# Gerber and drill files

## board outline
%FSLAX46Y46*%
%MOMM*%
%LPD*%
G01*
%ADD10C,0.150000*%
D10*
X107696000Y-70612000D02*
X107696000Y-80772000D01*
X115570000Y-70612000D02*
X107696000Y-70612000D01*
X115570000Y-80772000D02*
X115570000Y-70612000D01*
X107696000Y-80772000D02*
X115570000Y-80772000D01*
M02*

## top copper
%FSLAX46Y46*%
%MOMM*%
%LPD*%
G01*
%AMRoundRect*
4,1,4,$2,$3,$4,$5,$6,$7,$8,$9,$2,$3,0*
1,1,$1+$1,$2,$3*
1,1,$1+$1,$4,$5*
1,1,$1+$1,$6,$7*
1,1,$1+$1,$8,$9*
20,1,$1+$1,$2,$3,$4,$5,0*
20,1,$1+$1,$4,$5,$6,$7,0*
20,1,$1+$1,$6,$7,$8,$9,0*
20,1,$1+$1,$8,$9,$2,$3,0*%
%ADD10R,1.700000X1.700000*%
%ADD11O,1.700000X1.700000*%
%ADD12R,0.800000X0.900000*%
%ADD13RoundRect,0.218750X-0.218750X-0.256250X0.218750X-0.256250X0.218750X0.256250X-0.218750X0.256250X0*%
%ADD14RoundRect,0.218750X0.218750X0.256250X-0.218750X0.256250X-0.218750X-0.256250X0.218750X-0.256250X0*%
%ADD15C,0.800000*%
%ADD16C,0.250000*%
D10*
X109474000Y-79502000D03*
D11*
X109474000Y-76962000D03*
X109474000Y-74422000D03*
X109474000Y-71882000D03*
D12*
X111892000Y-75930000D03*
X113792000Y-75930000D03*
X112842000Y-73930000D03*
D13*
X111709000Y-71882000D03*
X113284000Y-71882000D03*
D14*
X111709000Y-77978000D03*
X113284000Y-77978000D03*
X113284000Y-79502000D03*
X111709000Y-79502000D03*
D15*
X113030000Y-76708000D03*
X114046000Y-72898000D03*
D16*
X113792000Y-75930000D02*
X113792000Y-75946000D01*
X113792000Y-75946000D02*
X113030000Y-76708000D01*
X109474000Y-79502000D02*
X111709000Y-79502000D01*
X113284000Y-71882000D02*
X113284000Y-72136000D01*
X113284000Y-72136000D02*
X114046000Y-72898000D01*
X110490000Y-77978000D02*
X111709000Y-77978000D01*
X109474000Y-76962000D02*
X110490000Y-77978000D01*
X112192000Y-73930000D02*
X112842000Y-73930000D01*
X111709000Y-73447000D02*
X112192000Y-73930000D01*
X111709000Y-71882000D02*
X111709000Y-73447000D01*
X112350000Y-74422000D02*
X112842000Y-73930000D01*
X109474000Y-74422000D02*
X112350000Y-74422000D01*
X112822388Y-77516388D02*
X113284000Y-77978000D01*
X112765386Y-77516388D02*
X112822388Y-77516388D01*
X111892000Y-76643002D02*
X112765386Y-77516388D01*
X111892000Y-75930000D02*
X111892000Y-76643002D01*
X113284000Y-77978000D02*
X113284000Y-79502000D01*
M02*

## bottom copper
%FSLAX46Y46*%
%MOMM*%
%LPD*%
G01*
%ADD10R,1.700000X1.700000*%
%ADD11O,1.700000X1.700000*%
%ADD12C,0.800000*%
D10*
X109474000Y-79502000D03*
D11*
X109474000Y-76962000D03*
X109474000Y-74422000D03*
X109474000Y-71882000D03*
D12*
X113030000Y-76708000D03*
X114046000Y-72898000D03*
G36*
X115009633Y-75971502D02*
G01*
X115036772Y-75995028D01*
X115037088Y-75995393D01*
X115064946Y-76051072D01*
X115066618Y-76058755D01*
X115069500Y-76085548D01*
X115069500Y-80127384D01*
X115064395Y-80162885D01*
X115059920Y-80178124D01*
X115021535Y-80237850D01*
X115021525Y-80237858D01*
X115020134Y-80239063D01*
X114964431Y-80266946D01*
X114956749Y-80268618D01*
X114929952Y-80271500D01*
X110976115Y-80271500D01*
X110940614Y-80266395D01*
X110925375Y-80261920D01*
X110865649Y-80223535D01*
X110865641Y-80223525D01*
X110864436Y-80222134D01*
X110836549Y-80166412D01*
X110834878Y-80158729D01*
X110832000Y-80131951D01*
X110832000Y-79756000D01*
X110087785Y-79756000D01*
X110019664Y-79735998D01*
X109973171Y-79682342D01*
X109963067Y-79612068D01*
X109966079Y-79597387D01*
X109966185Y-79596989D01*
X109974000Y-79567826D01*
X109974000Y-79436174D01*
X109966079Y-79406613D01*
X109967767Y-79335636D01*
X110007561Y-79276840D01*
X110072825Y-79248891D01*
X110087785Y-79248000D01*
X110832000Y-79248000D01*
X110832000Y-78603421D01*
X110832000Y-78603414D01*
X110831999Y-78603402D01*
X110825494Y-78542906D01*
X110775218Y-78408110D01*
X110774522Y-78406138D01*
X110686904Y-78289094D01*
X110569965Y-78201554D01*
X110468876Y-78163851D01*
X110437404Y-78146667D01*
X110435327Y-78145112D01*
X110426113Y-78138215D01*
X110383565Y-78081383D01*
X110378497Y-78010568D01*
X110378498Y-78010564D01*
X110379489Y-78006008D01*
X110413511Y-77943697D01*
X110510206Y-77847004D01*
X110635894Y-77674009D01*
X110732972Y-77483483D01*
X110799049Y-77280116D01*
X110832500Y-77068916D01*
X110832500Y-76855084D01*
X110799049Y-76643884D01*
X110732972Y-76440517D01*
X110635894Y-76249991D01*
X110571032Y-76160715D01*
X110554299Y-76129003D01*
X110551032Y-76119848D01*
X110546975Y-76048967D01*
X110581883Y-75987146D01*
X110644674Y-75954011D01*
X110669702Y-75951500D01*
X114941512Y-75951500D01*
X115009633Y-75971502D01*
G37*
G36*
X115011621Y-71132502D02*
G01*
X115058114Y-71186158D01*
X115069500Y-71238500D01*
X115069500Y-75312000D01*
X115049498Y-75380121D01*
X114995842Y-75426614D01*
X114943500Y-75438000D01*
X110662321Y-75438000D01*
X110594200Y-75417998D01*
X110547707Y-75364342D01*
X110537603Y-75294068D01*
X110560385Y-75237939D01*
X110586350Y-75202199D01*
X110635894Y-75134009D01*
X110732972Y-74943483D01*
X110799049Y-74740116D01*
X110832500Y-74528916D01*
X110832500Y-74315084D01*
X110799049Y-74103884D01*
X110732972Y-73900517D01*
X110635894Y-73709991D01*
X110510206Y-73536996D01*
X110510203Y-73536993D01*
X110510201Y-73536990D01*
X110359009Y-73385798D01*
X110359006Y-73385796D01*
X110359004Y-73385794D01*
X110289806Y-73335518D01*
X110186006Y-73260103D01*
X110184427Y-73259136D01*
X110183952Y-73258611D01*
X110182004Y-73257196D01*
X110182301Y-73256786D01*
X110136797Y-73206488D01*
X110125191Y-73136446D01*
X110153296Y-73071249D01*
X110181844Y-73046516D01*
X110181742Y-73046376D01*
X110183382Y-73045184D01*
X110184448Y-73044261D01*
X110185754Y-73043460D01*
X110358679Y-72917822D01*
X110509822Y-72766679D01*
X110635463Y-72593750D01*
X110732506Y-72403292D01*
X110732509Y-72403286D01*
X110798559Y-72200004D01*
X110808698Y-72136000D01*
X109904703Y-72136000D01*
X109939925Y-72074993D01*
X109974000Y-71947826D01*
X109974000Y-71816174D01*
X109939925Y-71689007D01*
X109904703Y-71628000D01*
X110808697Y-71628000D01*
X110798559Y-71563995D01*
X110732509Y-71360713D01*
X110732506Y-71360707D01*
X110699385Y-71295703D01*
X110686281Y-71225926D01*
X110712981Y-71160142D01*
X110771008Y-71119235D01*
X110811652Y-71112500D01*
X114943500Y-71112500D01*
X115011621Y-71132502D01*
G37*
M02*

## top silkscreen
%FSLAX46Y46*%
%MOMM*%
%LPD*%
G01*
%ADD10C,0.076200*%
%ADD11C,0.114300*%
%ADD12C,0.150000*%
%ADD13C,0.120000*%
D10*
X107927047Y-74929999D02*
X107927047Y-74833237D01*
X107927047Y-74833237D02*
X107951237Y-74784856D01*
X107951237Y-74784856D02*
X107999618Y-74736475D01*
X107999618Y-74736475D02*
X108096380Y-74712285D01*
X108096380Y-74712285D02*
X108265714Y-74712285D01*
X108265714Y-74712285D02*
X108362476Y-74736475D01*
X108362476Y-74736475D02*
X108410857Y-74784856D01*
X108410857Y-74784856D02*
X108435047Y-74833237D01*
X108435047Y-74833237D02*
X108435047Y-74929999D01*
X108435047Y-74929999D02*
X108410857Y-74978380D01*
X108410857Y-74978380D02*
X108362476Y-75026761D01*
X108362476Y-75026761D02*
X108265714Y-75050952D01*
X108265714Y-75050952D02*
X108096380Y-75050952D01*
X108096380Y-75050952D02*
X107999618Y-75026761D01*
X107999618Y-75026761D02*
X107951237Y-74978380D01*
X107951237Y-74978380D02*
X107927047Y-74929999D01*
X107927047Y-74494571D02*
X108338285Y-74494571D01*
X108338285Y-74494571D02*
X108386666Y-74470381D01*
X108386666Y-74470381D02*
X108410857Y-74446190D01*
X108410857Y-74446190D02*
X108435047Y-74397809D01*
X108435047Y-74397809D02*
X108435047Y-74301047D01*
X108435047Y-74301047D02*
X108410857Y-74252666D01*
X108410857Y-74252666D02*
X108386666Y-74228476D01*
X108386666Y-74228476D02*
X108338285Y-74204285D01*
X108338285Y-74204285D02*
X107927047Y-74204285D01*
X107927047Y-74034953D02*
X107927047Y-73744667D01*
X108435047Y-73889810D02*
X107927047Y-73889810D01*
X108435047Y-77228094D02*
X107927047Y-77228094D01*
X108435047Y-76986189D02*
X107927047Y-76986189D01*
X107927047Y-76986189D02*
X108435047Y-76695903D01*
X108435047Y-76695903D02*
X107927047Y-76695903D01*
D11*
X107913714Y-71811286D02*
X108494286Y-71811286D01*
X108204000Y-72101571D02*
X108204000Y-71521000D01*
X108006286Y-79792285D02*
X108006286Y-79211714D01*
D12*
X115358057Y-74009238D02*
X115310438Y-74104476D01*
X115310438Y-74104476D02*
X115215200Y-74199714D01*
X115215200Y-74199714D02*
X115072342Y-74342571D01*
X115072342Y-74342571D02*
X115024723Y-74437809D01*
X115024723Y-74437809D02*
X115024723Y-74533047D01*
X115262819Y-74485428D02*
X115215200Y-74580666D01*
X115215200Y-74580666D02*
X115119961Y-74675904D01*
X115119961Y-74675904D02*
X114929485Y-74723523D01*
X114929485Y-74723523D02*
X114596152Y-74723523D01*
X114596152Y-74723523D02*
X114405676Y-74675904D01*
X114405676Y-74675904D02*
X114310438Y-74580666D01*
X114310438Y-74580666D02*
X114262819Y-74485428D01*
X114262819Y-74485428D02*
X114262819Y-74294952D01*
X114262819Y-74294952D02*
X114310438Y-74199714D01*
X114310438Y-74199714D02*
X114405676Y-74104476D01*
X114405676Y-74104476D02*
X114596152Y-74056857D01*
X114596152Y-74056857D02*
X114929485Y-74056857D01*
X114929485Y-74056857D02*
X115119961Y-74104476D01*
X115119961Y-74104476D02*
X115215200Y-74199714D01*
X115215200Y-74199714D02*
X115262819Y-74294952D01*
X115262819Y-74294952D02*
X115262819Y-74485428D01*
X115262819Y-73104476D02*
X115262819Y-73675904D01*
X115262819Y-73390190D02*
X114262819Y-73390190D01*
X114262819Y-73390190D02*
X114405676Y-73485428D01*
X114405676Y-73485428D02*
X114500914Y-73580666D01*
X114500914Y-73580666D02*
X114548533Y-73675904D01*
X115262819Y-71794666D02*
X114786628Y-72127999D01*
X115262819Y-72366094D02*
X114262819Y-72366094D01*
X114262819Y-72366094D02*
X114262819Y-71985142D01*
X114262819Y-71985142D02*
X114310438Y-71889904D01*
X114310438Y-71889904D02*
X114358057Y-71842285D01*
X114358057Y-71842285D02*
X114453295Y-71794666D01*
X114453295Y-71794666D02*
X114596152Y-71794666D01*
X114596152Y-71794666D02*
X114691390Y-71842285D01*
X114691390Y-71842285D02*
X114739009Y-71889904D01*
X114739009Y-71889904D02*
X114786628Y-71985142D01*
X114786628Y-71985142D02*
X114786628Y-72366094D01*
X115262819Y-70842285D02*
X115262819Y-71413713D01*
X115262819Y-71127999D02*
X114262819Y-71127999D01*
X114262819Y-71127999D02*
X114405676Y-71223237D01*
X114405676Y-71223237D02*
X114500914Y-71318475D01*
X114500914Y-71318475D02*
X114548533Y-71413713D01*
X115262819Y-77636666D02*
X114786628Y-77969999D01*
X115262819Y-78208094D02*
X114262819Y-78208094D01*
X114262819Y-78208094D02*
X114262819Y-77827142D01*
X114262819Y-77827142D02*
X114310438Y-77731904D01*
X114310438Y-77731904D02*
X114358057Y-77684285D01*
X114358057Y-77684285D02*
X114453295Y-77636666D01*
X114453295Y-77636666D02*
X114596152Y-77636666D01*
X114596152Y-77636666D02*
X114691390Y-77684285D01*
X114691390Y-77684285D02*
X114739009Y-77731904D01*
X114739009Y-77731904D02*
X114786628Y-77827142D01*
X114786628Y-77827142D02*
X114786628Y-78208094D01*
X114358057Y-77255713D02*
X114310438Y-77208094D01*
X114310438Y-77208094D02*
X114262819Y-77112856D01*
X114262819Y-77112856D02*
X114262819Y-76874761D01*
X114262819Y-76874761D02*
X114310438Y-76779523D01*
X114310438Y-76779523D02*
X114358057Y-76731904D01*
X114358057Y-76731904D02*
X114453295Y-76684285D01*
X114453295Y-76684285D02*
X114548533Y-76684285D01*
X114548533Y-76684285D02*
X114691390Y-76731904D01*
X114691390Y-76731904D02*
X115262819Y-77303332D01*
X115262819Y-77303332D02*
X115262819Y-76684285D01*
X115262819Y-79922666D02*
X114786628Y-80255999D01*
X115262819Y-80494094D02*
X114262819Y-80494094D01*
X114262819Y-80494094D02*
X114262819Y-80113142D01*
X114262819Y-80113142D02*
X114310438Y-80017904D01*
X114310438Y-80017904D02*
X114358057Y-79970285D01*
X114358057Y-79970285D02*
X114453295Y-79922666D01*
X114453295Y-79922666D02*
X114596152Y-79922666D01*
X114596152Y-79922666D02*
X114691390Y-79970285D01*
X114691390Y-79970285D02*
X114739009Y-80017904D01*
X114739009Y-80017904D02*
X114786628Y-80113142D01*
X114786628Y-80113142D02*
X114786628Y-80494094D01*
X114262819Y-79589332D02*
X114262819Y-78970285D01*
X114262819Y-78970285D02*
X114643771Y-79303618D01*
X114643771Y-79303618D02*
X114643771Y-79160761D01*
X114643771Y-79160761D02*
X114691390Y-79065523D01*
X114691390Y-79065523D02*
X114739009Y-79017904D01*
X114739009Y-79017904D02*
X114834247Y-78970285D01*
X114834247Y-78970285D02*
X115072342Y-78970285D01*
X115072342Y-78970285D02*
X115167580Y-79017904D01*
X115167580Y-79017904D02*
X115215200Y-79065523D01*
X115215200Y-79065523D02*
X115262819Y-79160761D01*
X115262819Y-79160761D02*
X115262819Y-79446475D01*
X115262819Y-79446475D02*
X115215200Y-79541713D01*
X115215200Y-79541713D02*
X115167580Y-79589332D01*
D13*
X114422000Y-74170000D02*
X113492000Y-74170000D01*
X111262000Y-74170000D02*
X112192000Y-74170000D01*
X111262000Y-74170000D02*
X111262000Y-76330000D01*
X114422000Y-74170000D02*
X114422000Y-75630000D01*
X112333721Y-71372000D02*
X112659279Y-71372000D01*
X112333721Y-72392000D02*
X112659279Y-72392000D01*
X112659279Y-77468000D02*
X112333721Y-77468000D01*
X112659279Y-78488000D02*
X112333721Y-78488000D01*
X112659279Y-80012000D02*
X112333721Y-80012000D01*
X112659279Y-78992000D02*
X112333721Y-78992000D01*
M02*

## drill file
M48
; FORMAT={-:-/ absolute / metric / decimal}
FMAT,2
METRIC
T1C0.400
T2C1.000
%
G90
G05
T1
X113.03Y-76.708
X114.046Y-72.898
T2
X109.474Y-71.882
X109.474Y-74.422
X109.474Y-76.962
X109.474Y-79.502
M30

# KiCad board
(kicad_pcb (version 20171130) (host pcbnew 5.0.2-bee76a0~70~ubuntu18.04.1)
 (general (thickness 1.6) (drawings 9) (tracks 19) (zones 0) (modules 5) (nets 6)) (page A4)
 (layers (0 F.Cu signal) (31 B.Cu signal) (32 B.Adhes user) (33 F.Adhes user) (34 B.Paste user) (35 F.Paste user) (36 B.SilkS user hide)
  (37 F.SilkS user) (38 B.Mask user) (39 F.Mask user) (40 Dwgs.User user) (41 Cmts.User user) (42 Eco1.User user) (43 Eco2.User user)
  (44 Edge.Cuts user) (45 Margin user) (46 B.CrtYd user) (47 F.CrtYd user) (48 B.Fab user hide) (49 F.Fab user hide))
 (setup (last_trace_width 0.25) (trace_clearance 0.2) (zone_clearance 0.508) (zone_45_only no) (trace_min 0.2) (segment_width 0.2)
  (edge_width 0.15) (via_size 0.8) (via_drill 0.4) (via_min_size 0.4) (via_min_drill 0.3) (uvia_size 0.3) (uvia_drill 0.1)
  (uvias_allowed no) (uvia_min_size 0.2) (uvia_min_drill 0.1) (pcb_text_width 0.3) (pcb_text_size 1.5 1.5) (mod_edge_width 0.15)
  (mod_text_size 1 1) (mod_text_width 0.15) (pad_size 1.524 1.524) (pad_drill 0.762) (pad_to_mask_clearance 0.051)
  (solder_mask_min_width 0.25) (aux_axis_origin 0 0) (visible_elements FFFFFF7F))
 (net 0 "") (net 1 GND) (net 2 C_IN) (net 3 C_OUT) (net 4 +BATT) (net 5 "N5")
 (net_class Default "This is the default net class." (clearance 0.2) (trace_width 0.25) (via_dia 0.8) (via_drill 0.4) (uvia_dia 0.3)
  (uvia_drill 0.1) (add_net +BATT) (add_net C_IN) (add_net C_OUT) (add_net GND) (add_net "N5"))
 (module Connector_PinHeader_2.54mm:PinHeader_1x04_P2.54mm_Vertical (layer B.Cu) (at 109.474 79.502)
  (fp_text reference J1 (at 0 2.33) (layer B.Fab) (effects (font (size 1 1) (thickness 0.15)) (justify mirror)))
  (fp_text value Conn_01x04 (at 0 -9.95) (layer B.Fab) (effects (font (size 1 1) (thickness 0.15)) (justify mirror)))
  (pad 1 thru_hole rect (at 0 0) (size 1.7 1.7) (drill 1) (layers *.Cu *.Mask) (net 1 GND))
  (pad 2 thru_hole oval (at 0 -2.54) (size 1.7 1.7) (drill 1) (layers *.Cu *.Mask) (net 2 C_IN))
  (pad 3 thru_hole oval (at 0 -5.08) (size 1.7 1.7) (drill 1) (layers *.Cu *.Mask) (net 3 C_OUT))
  (pad 4 thru_hole oval (at 0 -7.62) (size 1.7 1.7) (drill 1) (layers *.Cu *.Mask) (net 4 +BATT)))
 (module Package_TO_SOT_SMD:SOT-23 (layer F.Cu) (at 112.842 74.93 90)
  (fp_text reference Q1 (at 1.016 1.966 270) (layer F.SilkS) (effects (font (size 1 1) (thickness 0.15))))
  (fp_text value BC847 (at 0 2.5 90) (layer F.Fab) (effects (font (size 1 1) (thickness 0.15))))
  (fp_line (start 0.76 1.58) (end 0.76 0.65) (layer F.SilkS) (width 0.12))
  (fp_line (start 0.76 -1.58) (end 0.76 -0.65) (layer F.SilkS) (width 0.12))
  (fp_line (start 0.76 -1.58) (end -1.4 -1.58) (layer F.SilkS) (width 0.12))
  (fp_line (start 0.76 1.58) (end -0.7 1.58) (layer F.SilkS) (width 0.12))
  (pad 1 smd rect (at -1 -0.95 90) (size 0.9 0.8) (layers F.Cu F.Paste F.Mask) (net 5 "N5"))
  (pad 2 smd rect (at -1 0.95 90) (size 0.9 0.8) (layers F.Cu F.Paste F.Mask) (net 1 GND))
  (pad 3 smd rect (at 1 0 90) (size 0.9 0.8) (layers F.Cu F.Paste F.Mask) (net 3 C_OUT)))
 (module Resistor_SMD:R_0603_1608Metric (layer F.Cu) (at 112.4965 71.882)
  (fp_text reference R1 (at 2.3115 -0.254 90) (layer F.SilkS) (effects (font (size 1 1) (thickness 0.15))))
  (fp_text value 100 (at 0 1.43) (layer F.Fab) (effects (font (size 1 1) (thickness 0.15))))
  (fp_line (start -0.162779 -0.51) (end 0.162779 -0.51) (layer F.SilkS) (width 0.12))
  (fp_line (start -0.162779 0.51) (end 0.162779 0.51) (layer F.SilkS) (width 0.12))
  (pad 1 smd roundrect (at -0.7875 0) (size 0.875 0.95) (layers F.Cu F.Paste F.Mask) (roundrect_rratio 0.25) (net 3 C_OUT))
  (pad 2 smd roundrect (at 0.7875 0) (size 0.875 0.95) (layers F.Cu F.Paste F.Mask) (roundrect_rratio 0.25) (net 4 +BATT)))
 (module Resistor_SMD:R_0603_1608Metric (layer F.Cu) (at 112.4965 77.978 180)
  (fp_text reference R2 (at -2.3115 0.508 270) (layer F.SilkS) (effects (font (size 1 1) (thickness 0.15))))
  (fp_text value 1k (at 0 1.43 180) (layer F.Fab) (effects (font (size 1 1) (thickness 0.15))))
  (fp_line (start -0.162779 0.51) (end 0.162779 0.51) (layer F.SilkS) (width 0.12))
  (fp_line (start -0.162779 -0.51) (end 0.162779 -0.51) (layer F.SilkS) (width 0.12))
  (pad 2 smd roundrect (at 0.7875 0 180) (size 0.875 0.95) (layers F.Cu F.Paste F.Mask) (roundrect_rratio 0.25) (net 2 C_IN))
  (pad 1 smd roundrect (at -0.7875 0 180) (size 0.875 0.95) (layers F.Cu F.Paste F.Mask) (roundrect_rratio 0.25) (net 5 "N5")))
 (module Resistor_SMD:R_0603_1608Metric (layer F.Cu) (at 112.4965 79.502 180)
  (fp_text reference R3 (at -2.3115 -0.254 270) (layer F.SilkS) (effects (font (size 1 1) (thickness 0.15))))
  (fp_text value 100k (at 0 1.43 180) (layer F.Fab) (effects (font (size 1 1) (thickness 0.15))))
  (fp_line (start -0.162779 -0.51) (end 0.162779 -0.51) (layer F.SilkS) (width 0.12))
  (fp_line (start -0.162779 0.51) (end 0.162779 0.51) (layer F.SilkS) (width 0.12))
  (pad 1 smd roundrect (at -0.7875 0 180) (size 0.875 0.95) (layers F.Cu F.Paste F.Mask) (roundrect_rratio 0.25) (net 5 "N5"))
  (pad 2 smd roundrect (at 0.7875 0 180) (size 0.875 0.95) (layers F.Cu F.Paste F.Mask) (roundrect_rratio 0.25) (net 1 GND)))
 (gr_line (start 107.696 70.612) (end 107.696 80.772) (layer Edge.Cuts) (width 0.15))
 (gr_line (start 115.57 70.612) (end 107.696 70.612) (layer Edge.Cuts) (width 0.15))
 (gr_line (start 115.57 80.772) (end 115.57 70.612) (layer Edge.Cuts) (width 0.15))
 (gr_line (start 107.696 80.772) (end 115.57 80.772) (layer Edge.Cuts) (width 0.15))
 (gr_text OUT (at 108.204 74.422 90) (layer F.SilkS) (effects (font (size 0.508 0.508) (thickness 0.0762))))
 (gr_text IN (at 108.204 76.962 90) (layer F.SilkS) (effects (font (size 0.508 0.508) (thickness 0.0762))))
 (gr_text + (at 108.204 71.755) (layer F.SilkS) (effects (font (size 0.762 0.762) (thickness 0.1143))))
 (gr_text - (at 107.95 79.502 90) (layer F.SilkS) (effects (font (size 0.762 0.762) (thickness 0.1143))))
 (via (at 113.03 76.708) (size 0.8) (drill 0.4) (layers F.Cu B.Cu) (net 1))
 (segment (start 113.792 75.93) (end 113.792 75.946) (width 0.25) (layer F.Cu) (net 1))
 (segment (start 113.792 75.946) (end 113.03 76.708) (width 0.25) (layer F.Cu) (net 1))
 (segment (start 109.474 79.502) (end 111.709 79.502) (width 0.25) (layer F.Cu) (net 1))
 (via (at 114.046 72.898) (size 0.8) (drill 0.4) (layers F.Cu B.Cu) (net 4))
 (segment (start 113.284 71.882) (end 113.284 72.136) (width 0.25) (layer F.Cu) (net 4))
 (segment (start 113.284 72.136) (end 114.046 72.898) (width 0.25) (layer F.Cu) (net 4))
 (segment (start 110.49 77.978) (end 111.709 77.978) (width 0.25) (layer F.Cu) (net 2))
 (segment (start 109.474 76.962) (end 110.49 77.978) (width 0.25) (layer F.Cu) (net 2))
 (segment (start 112.192 73.93) (end 112.842 73.93) (width 0.25) (layer F.Cu) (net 3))
 (segment (start 111.709 73.447) (end 112.192 73.93) (width 0.25) (layer F.Cu) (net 3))
 (segment (start 111.709 71.882) (end 111.709 73.447) (width 0.25) (layer F.Cu) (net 3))
 (segment (start 112.35 74.422) (end 112.842 73.93) (width 0.25) (layer F.Cu) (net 3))
 (segment (start 109.474 74.422) (end 112.35 74.422) (width 0.25) (layer F.Cu) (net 3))
 (segment (start 112.822388 77.516388) (end 113.284 77.978) (width 0.25) (layer F.Cu) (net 5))
 (segment (start 112.765386 77.516388) (end 112.822388 77.516388) (width 0.25) (layer F.Cu) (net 5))
 (segment (start 111.892 76.643002) (end 112.765386 77.516388) (width 0.25) (layer F.Cu) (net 5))
 (segment (start 111.892 75.93) (end 111.892 76.643002) (width 0.25) (layer F.Cu) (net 5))
 (segment (start 113.284 77.978) (end 113.284 79.502) (width 0.25) (layer F.Cu) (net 5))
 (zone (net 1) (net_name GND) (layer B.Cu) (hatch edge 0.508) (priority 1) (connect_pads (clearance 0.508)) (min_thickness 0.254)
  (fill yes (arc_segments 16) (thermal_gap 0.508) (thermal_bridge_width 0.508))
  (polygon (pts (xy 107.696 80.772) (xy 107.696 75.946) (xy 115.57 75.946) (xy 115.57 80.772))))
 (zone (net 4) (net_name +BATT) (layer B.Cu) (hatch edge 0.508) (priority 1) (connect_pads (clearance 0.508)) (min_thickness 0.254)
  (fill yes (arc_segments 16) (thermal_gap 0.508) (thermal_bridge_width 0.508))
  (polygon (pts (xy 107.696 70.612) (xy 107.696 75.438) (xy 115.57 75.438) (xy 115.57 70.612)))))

